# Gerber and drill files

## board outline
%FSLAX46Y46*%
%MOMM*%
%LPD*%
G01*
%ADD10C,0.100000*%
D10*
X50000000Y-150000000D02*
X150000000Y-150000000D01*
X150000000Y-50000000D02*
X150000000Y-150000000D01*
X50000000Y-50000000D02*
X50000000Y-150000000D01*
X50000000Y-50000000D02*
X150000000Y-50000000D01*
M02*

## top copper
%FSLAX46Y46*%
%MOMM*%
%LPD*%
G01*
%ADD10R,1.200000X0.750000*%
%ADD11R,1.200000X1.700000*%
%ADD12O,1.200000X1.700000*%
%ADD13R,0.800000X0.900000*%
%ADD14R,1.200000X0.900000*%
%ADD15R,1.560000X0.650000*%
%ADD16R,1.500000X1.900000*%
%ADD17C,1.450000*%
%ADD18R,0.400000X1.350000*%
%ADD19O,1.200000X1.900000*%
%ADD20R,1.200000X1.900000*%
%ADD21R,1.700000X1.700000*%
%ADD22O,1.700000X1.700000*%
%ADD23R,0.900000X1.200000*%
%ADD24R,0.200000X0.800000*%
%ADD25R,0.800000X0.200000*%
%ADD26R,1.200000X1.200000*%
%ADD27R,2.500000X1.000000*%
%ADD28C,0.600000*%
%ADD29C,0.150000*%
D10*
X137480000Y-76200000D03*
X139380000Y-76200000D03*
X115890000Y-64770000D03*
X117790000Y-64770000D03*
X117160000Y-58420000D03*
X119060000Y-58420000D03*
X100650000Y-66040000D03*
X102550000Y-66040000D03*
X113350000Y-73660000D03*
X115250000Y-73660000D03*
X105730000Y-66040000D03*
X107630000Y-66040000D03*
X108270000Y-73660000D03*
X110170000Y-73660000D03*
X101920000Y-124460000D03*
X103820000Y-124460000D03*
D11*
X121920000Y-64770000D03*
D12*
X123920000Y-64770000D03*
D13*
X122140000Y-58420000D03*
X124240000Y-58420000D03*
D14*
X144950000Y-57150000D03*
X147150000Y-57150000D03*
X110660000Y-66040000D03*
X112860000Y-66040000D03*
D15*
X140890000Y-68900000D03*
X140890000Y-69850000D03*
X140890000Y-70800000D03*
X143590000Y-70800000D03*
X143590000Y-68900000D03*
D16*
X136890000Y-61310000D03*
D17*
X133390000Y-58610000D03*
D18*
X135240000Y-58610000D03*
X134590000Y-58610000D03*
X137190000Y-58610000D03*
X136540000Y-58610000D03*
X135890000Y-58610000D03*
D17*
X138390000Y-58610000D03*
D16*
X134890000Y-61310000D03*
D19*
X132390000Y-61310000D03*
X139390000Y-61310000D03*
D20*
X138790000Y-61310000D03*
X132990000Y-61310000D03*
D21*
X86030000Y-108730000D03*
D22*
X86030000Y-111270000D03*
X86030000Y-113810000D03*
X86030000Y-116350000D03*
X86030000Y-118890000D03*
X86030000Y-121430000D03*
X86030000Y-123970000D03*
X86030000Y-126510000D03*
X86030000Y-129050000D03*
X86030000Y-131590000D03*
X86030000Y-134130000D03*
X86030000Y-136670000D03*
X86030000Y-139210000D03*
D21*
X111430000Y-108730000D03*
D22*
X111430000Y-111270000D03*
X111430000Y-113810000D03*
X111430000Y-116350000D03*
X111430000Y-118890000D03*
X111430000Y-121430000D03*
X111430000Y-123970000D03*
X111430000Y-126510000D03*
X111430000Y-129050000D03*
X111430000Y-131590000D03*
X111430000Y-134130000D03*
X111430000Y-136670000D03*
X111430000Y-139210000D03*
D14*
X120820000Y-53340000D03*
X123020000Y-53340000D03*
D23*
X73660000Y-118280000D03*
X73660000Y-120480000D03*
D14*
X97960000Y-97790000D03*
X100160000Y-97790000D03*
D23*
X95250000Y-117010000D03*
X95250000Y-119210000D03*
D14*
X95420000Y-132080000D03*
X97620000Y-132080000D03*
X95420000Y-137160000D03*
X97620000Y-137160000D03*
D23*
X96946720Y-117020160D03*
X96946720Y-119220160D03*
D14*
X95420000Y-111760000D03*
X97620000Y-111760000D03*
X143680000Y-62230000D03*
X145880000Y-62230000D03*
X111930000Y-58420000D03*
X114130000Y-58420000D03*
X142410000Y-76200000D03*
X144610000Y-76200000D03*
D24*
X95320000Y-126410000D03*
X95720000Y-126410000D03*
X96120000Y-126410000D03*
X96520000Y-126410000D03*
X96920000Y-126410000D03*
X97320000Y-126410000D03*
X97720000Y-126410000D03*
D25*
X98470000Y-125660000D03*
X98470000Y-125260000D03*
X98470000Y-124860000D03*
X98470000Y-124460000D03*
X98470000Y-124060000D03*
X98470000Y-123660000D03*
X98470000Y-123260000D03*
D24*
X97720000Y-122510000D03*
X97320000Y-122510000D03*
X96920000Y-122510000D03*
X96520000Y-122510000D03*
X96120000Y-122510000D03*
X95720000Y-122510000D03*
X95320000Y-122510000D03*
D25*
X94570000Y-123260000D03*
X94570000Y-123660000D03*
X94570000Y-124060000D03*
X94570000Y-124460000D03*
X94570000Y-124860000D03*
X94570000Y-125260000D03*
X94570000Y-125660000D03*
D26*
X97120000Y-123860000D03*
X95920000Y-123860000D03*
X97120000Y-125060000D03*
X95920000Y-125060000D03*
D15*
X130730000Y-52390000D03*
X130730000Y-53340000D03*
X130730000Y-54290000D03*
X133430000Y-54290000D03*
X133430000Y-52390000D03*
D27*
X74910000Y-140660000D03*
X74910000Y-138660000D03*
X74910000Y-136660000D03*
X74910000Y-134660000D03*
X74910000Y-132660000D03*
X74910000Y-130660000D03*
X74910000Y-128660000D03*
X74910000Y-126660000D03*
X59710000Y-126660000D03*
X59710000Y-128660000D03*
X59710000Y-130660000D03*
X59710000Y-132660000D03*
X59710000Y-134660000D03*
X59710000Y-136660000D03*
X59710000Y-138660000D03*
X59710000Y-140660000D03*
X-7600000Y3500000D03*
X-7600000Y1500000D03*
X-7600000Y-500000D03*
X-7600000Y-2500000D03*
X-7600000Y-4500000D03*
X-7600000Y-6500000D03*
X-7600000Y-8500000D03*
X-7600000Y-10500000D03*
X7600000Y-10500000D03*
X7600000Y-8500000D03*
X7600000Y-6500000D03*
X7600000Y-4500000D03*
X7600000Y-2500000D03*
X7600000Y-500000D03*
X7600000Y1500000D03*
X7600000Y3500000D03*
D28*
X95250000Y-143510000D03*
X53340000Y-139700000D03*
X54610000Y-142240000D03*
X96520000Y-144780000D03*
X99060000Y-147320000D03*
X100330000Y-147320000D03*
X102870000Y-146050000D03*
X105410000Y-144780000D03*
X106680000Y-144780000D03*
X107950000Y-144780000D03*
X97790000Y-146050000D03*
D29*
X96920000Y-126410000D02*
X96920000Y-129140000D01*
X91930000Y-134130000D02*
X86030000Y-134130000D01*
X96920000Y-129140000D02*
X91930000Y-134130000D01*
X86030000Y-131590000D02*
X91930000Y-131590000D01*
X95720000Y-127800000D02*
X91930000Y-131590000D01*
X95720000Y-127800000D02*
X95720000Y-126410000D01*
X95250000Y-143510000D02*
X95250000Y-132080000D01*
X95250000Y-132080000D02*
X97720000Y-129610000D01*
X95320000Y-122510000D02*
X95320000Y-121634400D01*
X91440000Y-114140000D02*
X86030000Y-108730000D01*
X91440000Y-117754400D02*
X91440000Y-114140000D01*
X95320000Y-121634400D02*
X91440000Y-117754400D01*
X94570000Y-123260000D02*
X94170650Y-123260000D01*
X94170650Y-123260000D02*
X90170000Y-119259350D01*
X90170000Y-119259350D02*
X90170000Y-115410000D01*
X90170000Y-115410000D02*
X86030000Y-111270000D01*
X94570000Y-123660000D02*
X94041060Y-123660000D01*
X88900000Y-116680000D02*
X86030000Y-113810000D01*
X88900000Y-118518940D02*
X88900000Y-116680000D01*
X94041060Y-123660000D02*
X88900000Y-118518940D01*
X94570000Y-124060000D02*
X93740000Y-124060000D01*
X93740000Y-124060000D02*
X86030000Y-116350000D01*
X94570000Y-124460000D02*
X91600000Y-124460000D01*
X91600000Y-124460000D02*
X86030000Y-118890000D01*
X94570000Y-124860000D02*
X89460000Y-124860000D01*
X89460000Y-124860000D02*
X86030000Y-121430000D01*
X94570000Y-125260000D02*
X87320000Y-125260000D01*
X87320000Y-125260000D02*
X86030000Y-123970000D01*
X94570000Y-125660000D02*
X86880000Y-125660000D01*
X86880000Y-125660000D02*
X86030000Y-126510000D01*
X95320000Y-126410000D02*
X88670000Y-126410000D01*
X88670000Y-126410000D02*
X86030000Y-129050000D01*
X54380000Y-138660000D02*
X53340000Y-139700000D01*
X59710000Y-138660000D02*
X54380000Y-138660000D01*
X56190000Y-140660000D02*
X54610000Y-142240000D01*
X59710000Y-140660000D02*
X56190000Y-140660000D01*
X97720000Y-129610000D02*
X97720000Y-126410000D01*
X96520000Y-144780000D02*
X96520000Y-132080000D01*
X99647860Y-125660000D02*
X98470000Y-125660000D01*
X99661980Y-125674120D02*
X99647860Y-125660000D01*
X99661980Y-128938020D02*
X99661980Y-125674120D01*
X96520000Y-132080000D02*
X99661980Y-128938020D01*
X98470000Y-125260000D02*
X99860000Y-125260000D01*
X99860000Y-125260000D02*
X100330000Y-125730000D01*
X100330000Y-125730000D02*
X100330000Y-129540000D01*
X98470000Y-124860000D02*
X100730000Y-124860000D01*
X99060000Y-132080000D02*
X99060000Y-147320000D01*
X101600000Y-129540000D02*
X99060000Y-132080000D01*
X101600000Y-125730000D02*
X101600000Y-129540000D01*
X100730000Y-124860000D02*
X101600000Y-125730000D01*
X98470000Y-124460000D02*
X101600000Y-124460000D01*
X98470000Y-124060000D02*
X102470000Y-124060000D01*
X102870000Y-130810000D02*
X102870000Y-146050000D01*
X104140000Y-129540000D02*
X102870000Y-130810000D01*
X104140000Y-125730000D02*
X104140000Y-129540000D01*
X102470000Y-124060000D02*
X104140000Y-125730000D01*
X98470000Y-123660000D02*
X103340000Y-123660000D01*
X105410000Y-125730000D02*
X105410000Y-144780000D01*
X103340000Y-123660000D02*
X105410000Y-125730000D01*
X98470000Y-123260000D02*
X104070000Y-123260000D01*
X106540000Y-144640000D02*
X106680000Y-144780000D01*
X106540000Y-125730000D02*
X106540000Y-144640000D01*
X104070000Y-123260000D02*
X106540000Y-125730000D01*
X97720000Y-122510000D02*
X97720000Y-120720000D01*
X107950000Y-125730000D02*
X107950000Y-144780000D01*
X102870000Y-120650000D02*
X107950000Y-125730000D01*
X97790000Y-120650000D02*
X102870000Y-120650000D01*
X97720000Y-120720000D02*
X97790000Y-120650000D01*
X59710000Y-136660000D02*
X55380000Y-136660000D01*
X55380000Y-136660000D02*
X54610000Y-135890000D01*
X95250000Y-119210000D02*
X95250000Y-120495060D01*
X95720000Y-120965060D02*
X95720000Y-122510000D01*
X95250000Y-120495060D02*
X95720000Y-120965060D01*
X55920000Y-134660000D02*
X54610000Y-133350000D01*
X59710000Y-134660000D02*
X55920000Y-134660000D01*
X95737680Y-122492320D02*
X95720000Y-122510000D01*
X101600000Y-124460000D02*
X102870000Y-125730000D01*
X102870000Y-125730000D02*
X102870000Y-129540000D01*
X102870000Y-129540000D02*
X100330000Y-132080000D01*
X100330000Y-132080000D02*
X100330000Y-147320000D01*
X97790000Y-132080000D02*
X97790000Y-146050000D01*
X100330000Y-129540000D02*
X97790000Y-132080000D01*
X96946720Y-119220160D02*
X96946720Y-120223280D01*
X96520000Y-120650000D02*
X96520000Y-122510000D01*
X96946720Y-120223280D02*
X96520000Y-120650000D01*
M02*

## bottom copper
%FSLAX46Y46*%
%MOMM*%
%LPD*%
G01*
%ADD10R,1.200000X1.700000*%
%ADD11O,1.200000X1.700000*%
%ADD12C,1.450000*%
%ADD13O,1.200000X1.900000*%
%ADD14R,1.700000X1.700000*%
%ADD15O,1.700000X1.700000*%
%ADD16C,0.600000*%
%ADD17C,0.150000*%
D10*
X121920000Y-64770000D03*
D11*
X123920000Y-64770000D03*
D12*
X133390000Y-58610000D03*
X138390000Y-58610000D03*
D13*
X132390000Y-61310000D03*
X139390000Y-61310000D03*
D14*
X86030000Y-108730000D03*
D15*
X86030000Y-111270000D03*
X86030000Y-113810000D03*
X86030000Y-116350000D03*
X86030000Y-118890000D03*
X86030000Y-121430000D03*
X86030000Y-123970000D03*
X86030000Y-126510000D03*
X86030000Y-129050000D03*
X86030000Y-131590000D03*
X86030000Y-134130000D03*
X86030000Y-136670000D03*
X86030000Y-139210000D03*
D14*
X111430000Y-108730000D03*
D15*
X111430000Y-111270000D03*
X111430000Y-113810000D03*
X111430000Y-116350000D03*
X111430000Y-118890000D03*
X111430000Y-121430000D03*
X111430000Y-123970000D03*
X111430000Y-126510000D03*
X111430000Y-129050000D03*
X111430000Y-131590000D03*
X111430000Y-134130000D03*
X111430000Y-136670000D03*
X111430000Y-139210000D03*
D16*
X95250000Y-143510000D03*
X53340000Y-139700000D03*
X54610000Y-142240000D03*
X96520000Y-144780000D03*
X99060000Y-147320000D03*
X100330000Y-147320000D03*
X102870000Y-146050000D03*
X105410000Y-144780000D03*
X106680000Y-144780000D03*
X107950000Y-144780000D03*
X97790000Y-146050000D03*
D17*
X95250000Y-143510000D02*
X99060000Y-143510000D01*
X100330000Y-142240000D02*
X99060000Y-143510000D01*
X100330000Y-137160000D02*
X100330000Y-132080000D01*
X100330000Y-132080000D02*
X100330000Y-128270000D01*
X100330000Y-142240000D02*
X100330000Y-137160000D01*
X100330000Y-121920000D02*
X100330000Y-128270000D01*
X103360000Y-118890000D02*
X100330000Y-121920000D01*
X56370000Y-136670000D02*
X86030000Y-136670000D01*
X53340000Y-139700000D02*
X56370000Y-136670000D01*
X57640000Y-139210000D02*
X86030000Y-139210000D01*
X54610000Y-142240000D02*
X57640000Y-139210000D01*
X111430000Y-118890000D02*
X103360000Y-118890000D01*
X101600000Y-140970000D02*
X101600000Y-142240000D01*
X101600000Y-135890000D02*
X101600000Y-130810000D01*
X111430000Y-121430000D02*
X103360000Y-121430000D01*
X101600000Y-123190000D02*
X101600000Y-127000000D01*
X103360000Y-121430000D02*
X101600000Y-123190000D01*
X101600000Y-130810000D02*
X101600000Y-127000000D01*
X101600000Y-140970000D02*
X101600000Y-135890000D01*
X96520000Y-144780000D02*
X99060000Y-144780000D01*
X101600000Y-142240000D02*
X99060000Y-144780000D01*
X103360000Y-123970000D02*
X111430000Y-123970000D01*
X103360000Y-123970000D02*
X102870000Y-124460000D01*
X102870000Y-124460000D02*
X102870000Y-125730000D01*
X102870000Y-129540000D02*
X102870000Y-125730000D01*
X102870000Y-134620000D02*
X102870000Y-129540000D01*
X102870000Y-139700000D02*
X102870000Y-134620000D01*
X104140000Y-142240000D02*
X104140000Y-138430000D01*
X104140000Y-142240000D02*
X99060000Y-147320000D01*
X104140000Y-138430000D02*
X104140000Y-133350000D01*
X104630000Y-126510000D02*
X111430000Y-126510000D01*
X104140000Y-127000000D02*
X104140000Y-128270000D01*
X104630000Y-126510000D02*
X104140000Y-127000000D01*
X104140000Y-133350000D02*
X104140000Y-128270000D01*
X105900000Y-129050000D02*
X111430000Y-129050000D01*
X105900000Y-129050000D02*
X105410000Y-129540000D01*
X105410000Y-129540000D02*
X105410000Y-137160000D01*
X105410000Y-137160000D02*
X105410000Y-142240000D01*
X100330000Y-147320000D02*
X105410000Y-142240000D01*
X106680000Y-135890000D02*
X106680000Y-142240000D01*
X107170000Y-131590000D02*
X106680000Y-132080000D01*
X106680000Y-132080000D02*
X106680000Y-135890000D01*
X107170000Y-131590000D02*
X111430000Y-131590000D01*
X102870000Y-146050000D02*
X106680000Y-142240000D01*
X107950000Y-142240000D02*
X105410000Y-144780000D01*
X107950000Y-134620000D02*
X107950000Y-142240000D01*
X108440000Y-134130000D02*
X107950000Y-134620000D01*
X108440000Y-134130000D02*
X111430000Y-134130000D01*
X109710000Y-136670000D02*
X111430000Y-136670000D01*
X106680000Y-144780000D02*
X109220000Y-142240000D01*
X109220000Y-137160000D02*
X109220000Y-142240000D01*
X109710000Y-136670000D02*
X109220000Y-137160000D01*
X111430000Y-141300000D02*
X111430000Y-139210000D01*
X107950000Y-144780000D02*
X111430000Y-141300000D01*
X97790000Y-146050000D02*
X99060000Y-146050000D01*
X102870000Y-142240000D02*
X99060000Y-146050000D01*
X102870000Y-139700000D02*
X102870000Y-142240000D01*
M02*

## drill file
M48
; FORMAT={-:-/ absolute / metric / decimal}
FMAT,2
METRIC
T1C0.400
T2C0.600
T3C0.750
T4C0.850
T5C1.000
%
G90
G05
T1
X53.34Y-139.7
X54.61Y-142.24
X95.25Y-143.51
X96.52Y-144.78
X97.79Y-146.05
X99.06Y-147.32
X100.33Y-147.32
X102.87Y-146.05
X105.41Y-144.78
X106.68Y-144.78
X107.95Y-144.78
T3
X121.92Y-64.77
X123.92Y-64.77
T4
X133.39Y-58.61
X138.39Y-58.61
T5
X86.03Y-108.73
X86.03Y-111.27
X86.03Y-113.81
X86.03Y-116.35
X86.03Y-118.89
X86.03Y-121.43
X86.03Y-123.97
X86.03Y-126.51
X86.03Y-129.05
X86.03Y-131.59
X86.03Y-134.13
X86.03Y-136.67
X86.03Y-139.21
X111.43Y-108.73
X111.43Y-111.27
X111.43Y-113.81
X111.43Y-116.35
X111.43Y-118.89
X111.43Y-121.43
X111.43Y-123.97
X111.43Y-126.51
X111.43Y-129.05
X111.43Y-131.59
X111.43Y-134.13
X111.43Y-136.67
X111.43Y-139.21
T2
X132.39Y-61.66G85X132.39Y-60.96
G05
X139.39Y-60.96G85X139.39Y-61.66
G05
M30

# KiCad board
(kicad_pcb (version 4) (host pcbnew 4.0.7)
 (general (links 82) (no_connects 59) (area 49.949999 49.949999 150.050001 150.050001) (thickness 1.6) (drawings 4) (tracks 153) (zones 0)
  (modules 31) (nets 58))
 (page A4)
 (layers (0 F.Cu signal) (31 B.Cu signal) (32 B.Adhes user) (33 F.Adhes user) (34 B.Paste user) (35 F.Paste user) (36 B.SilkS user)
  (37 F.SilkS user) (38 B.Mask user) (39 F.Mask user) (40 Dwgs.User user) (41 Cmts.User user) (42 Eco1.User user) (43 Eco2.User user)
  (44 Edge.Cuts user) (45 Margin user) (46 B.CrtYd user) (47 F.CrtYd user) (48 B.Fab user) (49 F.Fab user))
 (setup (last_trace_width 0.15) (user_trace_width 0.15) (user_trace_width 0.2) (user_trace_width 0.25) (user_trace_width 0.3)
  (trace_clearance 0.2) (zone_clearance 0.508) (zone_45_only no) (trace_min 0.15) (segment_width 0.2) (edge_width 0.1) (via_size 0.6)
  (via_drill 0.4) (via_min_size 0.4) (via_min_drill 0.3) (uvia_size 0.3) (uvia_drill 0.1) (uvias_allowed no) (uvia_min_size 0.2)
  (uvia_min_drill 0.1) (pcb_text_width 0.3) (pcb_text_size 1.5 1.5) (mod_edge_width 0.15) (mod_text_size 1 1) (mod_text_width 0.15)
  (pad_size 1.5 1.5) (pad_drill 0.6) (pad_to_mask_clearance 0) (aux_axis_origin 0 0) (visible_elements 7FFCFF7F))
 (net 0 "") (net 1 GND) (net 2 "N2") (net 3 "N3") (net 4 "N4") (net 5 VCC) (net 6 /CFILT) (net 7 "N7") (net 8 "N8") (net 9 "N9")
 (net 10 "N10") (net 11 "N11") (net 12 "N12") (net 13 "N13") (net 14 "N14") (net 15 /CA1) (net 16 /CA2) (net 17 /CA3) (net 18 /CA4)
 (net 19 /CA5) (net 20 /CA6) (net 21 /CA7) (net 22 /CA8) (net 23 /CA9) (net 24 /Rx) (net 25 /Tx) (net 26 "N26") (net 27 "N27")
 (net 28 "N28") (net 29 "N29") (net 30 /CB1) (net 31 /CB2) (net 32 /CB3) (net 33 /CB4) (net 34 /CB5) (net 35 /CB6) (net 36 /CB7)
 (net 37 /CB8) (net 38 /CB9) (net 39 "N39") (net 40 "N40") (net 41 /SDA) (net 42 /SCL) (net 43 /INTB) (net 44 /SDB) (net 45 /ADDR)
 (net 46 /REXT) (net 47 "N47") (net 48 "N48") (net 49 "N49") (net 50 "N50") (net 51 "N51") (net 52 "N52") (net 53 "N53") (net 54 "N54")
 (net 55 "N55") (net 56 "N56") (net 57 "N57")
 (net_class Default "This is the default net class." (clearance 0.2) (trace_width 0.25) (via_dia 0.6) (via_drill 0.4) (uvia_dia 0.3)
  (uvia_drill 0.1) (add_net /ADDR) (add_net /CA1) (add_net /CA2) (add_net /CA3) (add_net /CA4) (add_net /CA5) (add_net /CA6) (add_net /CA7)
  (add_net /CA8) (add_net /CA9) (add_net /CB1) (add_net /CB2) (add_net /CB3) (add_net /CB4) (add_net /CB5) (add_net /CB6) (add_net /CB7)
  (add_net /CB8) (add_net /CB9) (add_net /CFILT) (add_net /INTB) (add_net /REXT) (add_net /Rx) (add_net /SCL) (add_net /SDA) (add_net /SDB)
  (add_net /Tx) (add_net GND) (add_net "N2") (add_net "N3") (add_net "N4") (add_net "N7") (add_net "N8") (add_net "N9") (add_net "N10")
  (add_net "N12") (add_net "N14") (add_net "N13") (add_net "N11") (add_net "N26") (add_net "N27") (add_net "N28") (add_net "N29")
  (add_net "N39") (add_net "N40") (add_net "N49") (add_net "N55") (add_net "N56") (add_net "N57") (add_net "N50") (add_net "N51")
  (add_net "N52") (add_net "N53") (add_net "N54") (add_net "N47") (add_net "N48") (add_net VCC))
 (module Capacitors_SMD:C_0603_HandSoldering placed (layer F.Cu) (at 138.43 76.2)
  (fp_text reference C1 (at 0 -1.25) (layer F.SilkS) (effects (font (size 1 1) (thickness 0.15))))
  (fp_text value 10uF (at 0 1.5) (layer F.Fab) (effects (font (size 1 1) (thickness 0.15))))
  (pad 1 smd rect (at -0.95 0) (size 1.2 0.75) (layers F.Cu F.Paste F.Mask) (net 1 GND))
  (pad 2 smd rect (at 0.95 0) (size 1.2 0.75) (layers F.Cu F.Paste F.Mask) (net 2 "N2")))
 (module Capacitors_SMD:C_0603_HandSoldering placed (layer F.Cu) (at 116.84 64.77)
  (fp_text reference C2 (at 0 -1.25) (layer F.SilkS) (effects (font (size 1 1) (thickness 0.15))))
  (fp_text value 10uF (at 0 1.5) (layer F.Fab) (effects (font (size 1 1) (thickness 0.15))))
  (pad 1 smd rect (at -0.95 0) (size 1.2 0.75) (layers F.Cu F.Paste F.Mask) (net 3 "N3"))
  (pad 2 smd rect (at 0.95 0) (size 1.2 0.75) (layers F.Cu F.Paste F.Mask) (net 1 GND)))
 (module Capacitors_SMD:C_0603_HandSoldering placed (layer F.Cu) (at 118.11 58.42)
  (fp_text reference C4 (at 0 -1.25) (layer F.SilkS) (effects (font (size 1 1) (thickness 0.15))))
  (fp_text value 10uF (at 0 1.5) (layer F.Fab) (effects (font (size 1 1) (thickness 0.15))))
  (pad 1 smd rect (at -0.95 0) (size 1.2 0.75) (layers F.Cu F.Paste F.Mask) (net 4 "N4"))
  (pad 2 smd rect (at 0.95 0) (size 1.2 0.75) (layers F.Cu F.Paste F.Mask) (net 1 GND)))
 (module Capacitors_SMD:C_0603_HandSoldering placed (layer F.Cu) (at 101.6 66.04)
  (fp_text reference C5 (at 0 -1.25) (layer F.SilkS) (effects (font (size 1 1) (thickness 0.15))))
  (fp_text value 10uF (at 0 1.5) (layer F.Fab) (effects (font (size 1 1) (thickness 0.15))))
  (pad 1 smd rect (at -0.95 0) (size 1.2 0.75) (layers F.Cu F.Paste F.Mask) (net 1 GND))
  (pad 2 smd rect (at 0.95 0) (size 1.2 0.75) (layers F.Cu F.Paste F.Mask) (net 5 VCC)))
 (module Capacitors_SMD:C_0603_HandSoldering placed (layer F.Cu) (at 114.3 73.66)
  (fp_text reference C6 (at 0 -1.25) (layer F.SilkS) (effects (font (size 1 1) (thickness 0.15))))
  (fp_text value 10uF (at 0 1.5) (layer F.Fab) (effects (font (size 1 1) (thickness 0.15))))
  (pad 1 smd rect (at -0.95 0) (size 1.2 0.75) (layers F.Cu F.Paste F.Mask) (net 5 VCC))
  (pad 2 smd rect (at 0.95 0) (size 1.2 0.75) (layers F.Cu F.Paste F.Mask) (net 1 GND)))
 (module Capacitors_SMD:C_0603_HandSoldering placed (layer F.Cu) (at 106.68 66.04)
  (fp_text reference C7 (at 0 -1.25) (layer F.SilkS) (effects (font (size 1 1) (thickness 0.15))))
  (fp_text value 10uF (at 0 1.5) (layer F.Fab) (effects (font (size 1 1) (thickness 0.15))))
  (pad 1 smd rect (at -0.95 0) (size 1.2 0.75) (layers F.Cu F.Paste F.Mask) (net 5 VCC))
  (pad 2 smd rect (at 0.95 0) (size 1.2 0.75) (layers F.Cu F.Paste F.Mask) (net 1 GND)))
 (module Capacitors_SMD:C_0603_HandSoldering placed (layer F.Cu) (at 109.22 73.66)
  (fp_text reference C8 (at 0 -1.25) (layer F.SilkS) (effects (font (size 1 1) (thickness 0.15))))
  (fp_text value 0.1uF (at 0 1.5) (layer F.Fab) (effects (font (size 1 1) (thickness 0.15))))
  (pad 1 smd rect (at -0.95 0) (size 1.2 0.75) (layers F.Cu F.Paste F.Mask) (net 5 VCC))
  (pad 2 smd rect (at 0.95 0) (size 1.2 0.75) (layers F.Cu F.Paste F.Mask) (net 1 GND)))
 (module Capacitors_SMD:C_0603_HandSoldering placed (layer F.Cu) (at 102.87 124.46)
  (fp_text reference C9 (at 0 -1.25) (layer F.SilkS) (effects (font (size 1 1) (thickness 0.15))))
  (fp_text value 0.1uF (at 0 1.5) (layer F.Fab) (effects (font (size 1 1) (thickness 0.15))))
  (pad 1 smd rect (at -0.95 0) (size 1.2 0.75) (layers F.Cu F.Paste F.Mask) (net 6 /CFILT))
  (pad 2 smd rect (at 0.95 0) (size 1.2 0.75) (layers F.Cu F.Paste F.Mask) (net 1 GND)))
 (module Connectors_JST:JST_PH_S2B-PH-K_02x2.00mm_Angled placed (layer F.Cu) (at 121.92 64.77)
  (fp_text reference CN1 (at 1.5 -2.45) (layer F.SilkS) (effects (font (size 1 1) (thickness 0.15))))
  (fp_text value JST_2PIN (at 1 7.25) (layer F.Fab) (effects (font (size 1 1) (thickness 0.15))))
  (pad 1 thru_hole rect (at 0 0) (size 1.2 1.7) (drill 0.75) (layers *.Cu *.Mask) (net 1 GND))
  (pad 2 thru_hole oval (at 2 0) (size 1.2 1.7) (drill 0.75) (layers *.Cu *.Mask) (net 3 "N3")))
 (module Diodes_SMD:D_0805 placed (layer F.Cu) (at 123.19 58.42)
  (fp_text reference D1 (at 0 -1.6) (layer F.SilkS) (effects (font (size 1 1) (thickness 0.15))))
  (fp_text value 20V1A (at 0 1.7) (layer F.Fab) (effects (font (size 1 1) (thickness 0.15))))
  (pad 1 smd rect (at -1.05 0) (size 0.8 0.9) (layers F.Cu F.Paste F.Mask) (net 4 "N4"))
  (pad 2 smd rect (at 1.05 0) (size 0.8 0.9) (layers F.Cu F.Paste F.Mask) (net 3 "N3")))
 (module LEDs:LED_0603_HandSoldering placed (layer F.Cu) (at 146.05 57.15)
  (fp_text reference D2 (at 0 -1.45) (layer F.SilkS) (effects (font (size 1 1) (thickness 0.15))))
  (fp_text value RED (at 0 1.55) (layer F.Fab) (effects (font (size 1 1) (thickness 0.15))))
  (pad 1 smd rect (at -1.1 0) (size 1.2 0.9) (layers F.Cu F.Paste F.Mask) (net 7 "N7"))
  (pad 2 smd rect (at 1.1 0) (size 1.2 0.9) (layers F.Cu F.Paste F.Mask) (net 2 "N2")))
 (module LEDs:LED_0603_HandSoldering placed (layer F.Cu) (at 111.76 66.04)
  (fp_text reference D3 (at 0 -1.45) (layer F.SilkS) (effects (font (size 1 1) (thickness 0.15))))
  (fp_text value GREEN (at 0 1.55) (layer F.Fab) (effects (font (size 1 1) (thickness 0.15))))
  (pad 1 smd rect (at -1.1 0) (size 1.2 0.9) (layers F.Cu F.Paste F.Mask) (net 1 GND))
  (pad 2 smd rect (at 1.1 0) (size 1.2 0.9) (layers F.Cu F.Paste F.Mask) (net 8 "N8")))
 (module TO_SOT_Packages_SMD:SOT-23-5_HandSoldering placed (layer F.Cu) (at 142.24 69.85)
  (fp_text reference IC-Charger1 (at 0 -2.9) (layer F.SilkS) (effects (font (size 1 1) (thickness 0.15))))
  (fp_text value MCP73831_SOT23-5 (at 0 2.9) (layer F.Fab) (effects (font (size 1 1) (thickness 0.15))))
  (pad 1 smd rect (at -1.35 -0.95) (size 1.56 0.65) (layers F.Cu F.Paste F.Mask) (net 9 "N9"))
  (pad 2 smd rect (at -1.35 0) (size 1.56 0.65) (layers F.Cu F.Paste F.Mask) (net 1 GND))
  (pad 3 smd rect (at -1.35 0.95) (size 1.56 0.65) (layers F.Cu F.Paste F.Mask) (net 3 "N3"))
  (pad 4 smd rect (at 1.35 0.95) (size 1.56 0.65) (layers F.Cu F.Paste F.Mask) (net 2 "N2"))
  (pad 5 smd rect (at 1.35 -0.95) (size 1.56 0.65) (layers F.Cu F.Paste F.Mask) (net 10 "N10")))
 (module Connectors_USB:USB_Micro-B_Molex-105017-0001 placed (layer F.Cu) (at 135.89 60.96)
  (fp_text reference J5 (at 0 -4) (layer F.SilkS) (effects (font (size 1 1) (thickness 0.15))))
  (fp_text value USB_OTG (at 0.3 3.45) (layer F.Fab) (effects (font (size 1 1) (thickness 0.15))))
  (pad 6 smd rect (at 1 0.35) (size 1.5 1.9) (layers F.Cu F.Paste F.Mask) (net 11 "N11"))
  (pad 6 thru_hole circle (at -2.5 -2.35) (size 1.45 1.45) (drill 0.85) (layers *.Cu *.Mask) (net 11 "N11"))
  (pad 2 smd rect (at -0.65 -2.35) (size 0.4 1.35) (layers F.Cu F.Paste F.Mask) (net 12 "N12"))
  (pad 1 smd rect (at -1.3 -2.35) (size 0.4 1.35) (layers F.Cu F.Paste F.Mask) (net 2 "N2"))
  (pad 5 smd rect (at 1.3 -2.35) (size 0.4 1.35) (layers F.Cu F.Paste F.Mask) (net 1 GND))
  (pad 4 smd rect (at 0.65 -2.35) (size 0.4 1.35) (layers F.Cu F.Paste F.Mask) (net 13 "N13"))
  (pad 3 smd rect (at 0 -2.35) (size 0.4 1.35) (layers F.Cu F.Paste F.Mask) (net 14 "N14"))
  (pad 6 thru_hole circle (at 2.5 -2.35) (size 1.45 1.45) (drill 0.85) (layers *.Cu *.Mask) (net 11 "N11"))
  (pad 6 smd rect (at -1 0.35) (size 1.5 1.9) (layers F.Cu F.Paste F.Mask) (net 11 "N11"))
  (pad 6 thru_hole oval (at -3.5 0.35 180) (size 1.2 1.9) (drill oval 0.6 1.3) (layers *.Cu *.Mask) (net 11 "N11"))
  (pad 6 thru_hole oval (at 3.5 0.35) (size 1.2 1.9) (drill oval 0.6 1.3) (layers *.Cu *.Mask) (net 11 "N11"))
  (pad 6 smd rect (at 2.9 0.35) (size 1.2 1.9) (layers F.Cu F.Mask) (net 11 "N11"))
  (pad 6 smd rect (at -2.9 0.35) (size 1.2 1.9) (layers F.Cu F.Mask) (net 11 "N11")))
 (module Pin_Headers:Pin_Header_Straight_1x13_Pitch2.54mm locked (layer F.Cu) (at 86.03 108.73)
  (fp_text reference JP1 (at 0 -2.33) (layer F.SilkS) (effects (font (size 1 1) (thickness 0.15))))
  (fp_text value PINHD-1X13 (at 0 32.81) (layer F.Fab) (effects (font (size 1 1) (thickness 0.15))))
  (pad 1 thru_hole rect (at 0 0) (size 1.7 1.7) (drill 1) (layers *.Cu *.Mask) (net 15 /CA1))
  (pad 2 thru_hole oval (at 0 2.54) (size 1.7 1.7) (drill 1) (layers *.Cu *.Mask) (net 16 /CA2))
  (pad 3 thru_hole oval (at 0 5.08) (size 1.7 1.7) (drill 1) (layers *.Cu *.Mask) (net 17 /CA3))
  (pad 4 thru_hole oval (at 0 7.62) (size 1.7 1.7) (drill 1) (layers *.Cu *.Mask) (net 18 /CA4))
  (pad 5 thru_hole oval (at 0 10.16) (size 1.7 1.7) (drill 1) (layers *.Cu *.Mask) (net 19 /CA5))
  (pad 6 thru_hole oval (at 0 12.7) (size 1.7 1.7) (drill 1) (layers *.Cu *.Mask) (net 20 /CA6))
  (pad 7 thru_hole oval (at 0 15.24) (size 1.7 1.7) (drill 1) (layers *.Cu *.Mask) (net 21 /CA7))
  (pad 8 thru_hole oval (at 0 17.78) (size 1.7 1.7) (drill 1) (layers *.Cu *.Mask) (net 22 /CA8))
  (pad 9 thru_hole oval (at 0 20.32) (size 1.7 1.7) (drill 1) (layers *.Cu *.Mask) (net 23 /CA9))
  (pad 10 thru_hole oval (at 0 22.86) (size 1.7 1.7) (drill 1) (layers *.Cu *.Mask) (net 5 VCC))
  (pad 11 thru_hole oval (at 0 25.4) (size 1.7 1.7) (drill 1) (layers *.Cu *.Mask) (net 1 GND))
  (pad 12 thru_hole oval (at 0 27.94) (size 1.7 1.7) (drill 1) (layers *.Cu *.Mask) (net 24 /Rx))
  (pad 13 thru_hole oval (at 0 30.48) (size 1.7 1.7) (drill 1) (layers *.Cu *.Mask) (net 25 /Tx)))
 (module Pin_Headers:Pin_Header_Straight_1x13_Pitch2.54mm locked (layer F.Cu) (at 111.43 108.73)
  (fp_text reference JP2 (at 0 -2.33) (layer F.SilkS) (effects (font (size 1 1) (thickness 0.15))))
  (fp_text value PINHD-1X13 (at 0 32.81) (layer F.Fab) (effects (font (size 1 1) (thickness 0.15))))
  (pad 1 thru_hole rect (at 0 0) (size 1.7 1.7) (drill 1) (layers *.Cu *.Mask) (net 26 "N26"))
  (pad 2 thru_hole oval (at 0 2.54) (size 1.7 1.7) (drill 1) (layers *.Cu *.Mask) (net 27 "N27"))
  (pad 3 thru_hole oval (at 0 5.08) (size 1.7 1.7) (drill 1) (layers *.Cu *.Mask) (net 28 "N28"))
  (pad 4 thru_hole oval (at 0 7.62) (size 1.7 1.7) (drill 1) (layers *.Cu *.Mask) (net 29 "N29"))
  (pad 5 thru_hole oval (at 0 10.16) (size 1.7 1.7) (drill 1) (layers *.Cu *.Mask) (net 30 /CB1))
  (pad 6 thru_hole oval (at 0 12.7) (size 1.7 1.7) (drill 1) (layers *.Cu *.Mask) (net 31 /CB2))
  (pad 7 thru_hole oval (at 0 15.24) (size 1.7 1.7) (drill 1) (layers *.Cu *.Mask) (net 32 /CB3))
  (pad 8 thru_hole oval (at 0 17.78) (size 1.7 1.7) (drill 1) (layers *.Cu *.Mask) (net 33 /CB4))
  (pad 9 thru_hole oval (at 0 20.32) (size 1.7 1.7) (drill 1) (layers *.Cu *.Mask) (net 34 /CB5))
  (pad 10 thru_hole oval (at 0 22.86) (size 1.7 1.7) (drill 1) (layers *.Cu *.Mask) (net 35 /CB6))
  (pad 11 thru_hole oval (at 0 25.4) (size 1.7 1.7) (drill 1) (layers *.Cu *.Mask) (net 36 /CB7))
  (pad 12 thru_hole oval (at 0 27.94) (size 1.7 1.7) (drill 1) (layers *.Cu *.Mask) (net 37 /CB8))
  (pad 13 thru_hole oval (at 0 30.48) (size 1.7 1.7) (drill 1) (layers *.Cu *.Mask) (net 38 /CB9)))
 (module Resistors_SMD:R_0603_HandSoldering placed (layer F.Cu) (at 121.92 53.34)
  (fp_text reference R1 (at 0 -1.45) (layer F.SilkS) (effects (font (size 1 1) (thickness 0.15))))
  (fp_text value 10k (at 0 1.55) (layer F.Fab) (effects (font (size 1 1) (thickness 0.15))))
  (pad 1 smd rect (at -1.1 0) (size 1.2 0.9) (layers F.Cu F.Paste F.Mask) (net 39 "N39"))
  (pad 2 smd rect (at 1.1 0) (size 1.2 0.9) (layers F.Cu F.Paste F.Mask) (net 4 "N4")))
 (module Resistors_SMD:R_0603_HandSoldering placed (layer F.Cu) (at 73.66 119.38 270)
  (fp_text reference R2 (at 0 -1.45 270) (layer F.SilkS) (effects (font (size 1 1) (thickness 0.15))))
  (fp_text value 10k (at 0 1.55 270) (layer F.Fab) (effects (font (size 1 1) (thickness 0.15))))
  (pad 1 smd rect (at -1.1 0 270) (size 1.2 0.9) (layers F.Cu F.Paste F.Mask) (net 5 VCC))
  (pad 2 smd rect (at 1.1 0 270) (size 1.2 0.9) (layers F.Cu F.Paste F.Mask) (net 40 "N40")))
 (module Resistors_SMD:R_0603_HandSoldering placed (layer F.Cu) (at 99.06 97.79)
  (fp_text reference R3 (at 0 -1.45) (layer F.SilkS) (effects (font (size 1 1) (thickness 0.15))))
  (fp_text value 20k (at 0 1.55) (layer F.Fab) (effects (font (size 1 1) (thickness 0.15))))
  (pad 1 smd rect (at -1.1 0) (size 1.2 0.9) (layers F.Cu F.Paste F.Mask) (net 5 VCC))
  (pad 2 smd rect (at 1.1 0) (size 1.2 0.9) (layers F.Cu F.Paste F.Mask) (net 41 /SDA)))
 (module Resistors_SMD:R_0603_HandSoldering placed (layer F.Cu) (at 95.25 118.11 270)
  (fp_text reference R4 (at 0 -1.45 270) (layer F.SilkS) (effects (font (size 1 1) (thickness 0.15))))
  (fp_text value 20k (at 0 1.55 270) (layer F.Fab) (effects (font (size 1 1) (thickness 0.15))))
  (pad 1 smd rect (at -1.1 0 270) (size 1.2 0.9) (layers F.Cu F.Paste F.Mask) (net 5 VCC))
  (pad 2 smd rect (at 1.1 0 270) (size 1.2 0.9) (layers F.Cu F.Paste F.Mask) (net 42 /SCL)))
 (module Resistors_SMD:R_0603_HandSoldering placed (layer F.Cu) (at 96.52 132.08)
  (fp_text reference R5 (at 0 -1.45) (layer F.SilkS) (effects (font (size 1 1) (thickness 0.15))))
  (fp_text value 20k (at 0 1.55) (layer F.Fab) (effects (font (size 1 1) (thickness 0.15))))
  (pad 1 smd rect (at -1.1 0) (size 1.2 0.9) (layers F.Cu F.Paste F.Mask) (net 5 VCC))
  (pad 2 smd rect (at 1.1 0) (size 1.2 0.9) (layers F.Cu F.Paste F.Mask) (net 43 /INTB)))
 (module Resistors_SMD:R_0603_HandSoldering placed (layer F.Cu) (at 96.52 137.16)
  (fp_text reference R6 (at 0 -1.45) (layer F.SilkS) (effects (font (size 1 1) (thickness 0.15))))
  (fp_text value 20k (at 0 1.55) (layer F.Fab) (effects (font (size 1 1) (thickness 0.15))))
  (pad 1 smd rect (at -1.1 0) (size 1.2 0.9) (layers F.Cu F.Paste F.Mask) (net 5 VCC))
  (pad 2 smd rect (at 1.1 0) (size 1.2 0.9) (layers F.Cu F.Paste F.Mask) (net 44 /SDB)))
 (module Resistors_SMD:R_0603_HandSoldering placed (layer F.Cu) (at 96.94672 118.12016 270)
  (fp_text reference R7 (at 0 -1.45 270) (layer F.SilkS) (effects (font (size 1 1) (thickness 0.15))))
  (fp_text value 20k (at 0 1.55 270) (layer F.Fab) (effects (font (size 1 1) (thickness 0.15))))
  (pad 1 smd rect (at -1.1 0 270) (size 1.2 0.9) (layers F.Cu F.Paste F.Mask) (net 1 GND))
  (pad 2 smd rect (at 1.1 0 270) (size 1.2 0.9) (layers F.Cu F.Paste F.Mask) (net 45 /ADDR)))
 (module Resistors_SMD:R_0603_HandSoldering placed (layer F.Cu) (at 96.52 111.76)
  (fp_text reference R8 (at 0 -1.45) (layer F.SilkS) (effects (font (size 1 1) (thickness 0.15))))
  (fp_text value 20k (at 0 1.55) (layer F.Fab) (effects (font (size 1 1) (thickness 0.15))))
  (pad 1 smd rect (at -1.1 0) (size 1.2 0.9) (layers F.Cu F.Paste F.Mask) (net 1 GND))
  (pad 2 smd rect (at 1.1 0) (size 1.2 0.9) (layers F.Cu F.Paste F.Mask) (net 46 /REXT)))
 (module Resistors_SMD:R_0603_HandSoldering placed (layer F.Cu) (at 144.78 62.23)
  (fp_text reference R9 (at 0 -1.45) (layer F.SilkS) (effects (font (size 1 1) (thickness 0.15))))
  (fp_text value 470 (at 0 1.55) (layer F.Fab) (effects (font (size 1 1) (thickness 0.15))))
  (pad 1 smd rect (at -1.1 0) (size 1.2 0.9) (layers F.Cu F.Paste F.Mask) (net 9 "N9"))
  (pad 2 smd rect (at 1.1 0) (size 1.2 0.9) (layers F.Cu F.Paste F.Mask) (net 7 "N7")))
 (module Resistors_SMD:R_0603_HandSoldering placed (layer F.Cu) (at 113.03 58.42)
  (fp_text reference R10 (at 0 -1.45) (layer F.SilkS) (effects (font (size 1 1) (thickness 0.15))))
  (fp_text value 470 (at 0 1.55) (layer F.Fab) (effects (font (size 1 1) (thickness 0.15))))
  (pad 1 smd rect (at -1.1 0) (size 1.2 0.9) (layers F.Cu F.Paste F.Mask) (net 9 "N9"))
  (pad 2 smd rect (at 1.1 0) (size 1.2 0.9) (layers F.Cu F.Paste F.Mask) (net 8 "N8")))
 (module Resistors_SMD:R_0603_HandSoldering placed (layer F.Cu) (at 143.51 76.2)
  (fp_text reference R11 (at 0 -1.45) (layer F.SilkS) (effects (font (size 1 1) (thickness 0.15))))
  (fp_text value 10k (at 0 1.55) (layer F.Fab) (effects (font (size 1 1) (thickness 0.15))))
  (pad 1 smd rect (at -1.1 0) (size 1.2 0.9) (layers F.Cu F.Paste F.Mask) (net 1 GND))
  (pad 2 smd rect (at 1.1 0) (size 1.2 0.9) (layers F.Cu F.Paste F.Mask) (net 10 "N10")))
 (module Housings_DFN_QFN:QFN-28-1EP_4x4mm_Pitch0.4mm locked (layer F.Cu) (at 96.52 124.46 90)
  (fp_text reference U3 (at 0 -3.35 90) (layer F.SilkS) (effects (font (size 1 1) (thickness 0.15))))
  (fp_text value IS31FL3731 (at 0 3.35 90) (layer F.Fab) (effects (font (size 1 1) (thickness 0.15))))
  (pad 1 smd rect (at -1.95 -1.2 90) (size 0.8 0.2) (layers F.Cu F.Paste F.Mask) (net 23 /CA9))
  (pad 2 smd rect (at -1.95 -0.8 90) (size 0.8 0.2) (layers F.Cu F.Paste F.Mask) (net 5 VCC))
  (pad 3 smd rect (at -1.95 -0.4 90) (size 0.8 0.2) (layers F.Cu F.Paste F.Mask) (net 44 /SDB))
  (pad 4 smd rect (at -1.95 0 90) (size 0.8 0.2) (layers F.Cu F.Paste F.Mask) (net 43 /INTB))
  (pad 5 smd rect (at -1.95 0.4 90) (size 0.8 0.2) (layers F.Cu F.Paste F.Mask) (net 1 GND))
  (pad 6 smd rect (at -1.95 0.8 90) (size 0.8 0.2) (layers F.Cu F.Paste F.Mask) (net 46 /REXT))
  (pad 7 smd rect (at -1.95 1.2 90) (size 0.8 0.2) (layers F.Cu F.Paste F.Mask) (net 30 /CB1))
  (pad 8 smd rect (at -1.2 1.95 180) (size 0.8 0.2) (layers F.Cu F.Paste F.Mask) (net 31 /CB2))
  (pad 9 smd rect (at -0.8 1.95 180) (size 0.8 0.2) (layers F.Cu F.Paste F.Mask) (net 32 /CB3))
  (pad 10 smd rect (at -0.4 1.95 180) (size 0.8 0.2) (layers F.Cu F.Paste F.Mask) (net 33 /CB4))
  (pad 11 smd rect (at 0 1.95 180) (size 0.8 0.2) (layers F.Cu F.Paste F.Mask) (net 34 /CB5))
  (pad 12 smd rect (at 0.4 1.95 180) (size 0.8 0.2) (layers F.Cu F.Paste F.Mask) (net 35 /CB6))
  (pad 13 smd rect (at 0.8 1.95 180) (size 0.8 0.2) (layers F.Cu F.Paste F.Mask) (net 36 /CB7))
  (pad 14 smd rect (at 1.2 1.95 180) (size 0.8 0.2) (layers F.Cu F.Paste F.Mask) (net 37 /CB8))
  (pad 15 smd rect (at 1.95 1.2 90) (size 0.8 0.2) (layers F.Cu F.Paste F.Mask) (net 38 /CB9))
  (pad 16 smd rect (at 1.95 0.8 90) (size 0.8 0.2) (layers F.Cu F.Paste F.Mask) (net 6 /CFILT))
  (pad 17 smd rect (at 1.95 0.4 90) (size 0.8 0.2) (layers F.Cu F.Paste F.Mask) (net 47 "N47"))
  (pad 18 smd rect (at 1.95 0 90) (size 0.8 0.2) (layers F.Cu F.Paste F.Mask) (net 45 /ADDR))
  (pad 19 smd rect (at 1.95 -0.4 90) (size 0.8 0.2) (layers F.Cu F.Paste F.Mask) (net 41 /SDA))
  (pad 20 smd rect (at 1.95 -0.8 90) (size 0.8 0.2) (layers F.Cu F.Paste F.Mask) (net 42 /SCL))
  (pad 21 smd rect (at 1.95 -1.2 90) (size 0.8 0.2) (layers F.Cu F.Paste F.Mask) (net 15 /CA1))
  (pad 22 smd rect (at 1.2 -1.95 180) (size 0.8 0.2) (layers F.Cu F.Paste F.Mask) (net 16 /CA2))
  (pad 23 smd rect (at 0.8 -1.95 180) (size 0.8 0.2) (layers F.Cu F.Paste F.Mask) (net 17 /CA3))
  (pad 24 smd rect (at 0.4 -1.95 180) (size 0.8 0.2) (layers F.Cu F.Paste F.Mask) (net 18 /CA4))
  (pad 25 smd rect (at 0 -1.95 180) (size 0.8 0.2) (layers F.Cu F.Paste F.Mask) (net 19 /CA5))
  (pad 26 smd rect (at -0.4 -1.95 180) (size 0.8 0.2) (layers F.Cu F.Paste F.Mask) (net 20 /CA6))
  (pad 27 smd rect (at -0.8 -1.95 180) (size 0.8 0.2) (layers F.Cu F.Paste F.Mask) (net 21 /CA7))
  (pad 28 smd rect (at -1.2 -1.95 180) (size 0.8 0.2) (layers F.Cu F.Paste F.Mask) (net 22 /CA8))
  (pad 29 smd rect (at 0.6 0.6 90) (size 1.2 1.2) (layers F.Cu F.Paste F.Mask) (solder_paste_margin_ratio -0.2))
  (pad 29 smd rect (at 0.6 -0.6 90) (size 1.2 1.2) (layers F.Cu F.Paste F.Mask) (solder_paste_margin_ratio -0.2))
  (pad 29 smd rect (at -0.6 0.6 90) (size 1.2 1.2) (layers F.Cu F.Paste F.Mask) (solder_paste_margin_ratio -0.2))
  (pad 29 smd rect (at -0.6 -0.6 90) (size 1.2 1.2) (layers F.Cu F.Paste F.Mask) (solder_paste_margin_ratio -0.2)))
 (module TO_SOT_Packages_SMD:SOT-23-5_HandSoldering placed (layer F.Cu) (at 132.08 53.34)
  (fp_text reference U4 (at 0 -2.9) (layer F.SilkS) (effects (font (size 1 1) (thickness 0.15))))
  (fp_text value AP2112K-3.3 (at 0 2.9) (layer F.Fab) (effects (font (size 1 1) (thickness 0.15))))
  (pad 1 smd rect (at -1.35 -0.95) (size 1.56 0.65) (layers F.Cu F.Paste F.Mask) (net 4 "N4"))
  (pad 2 smd rect (at -1.35 0) (size 1.56 0.65) (layers F.Cu F.Paste F.Mask) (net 1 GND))
  (pad 3 smd rect (at -1.35 0.95) (size 1.56 0.65) (layers F.Cu F.Paste F.Mask) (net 39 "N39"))
  (pad 4 smd rect (at 1.35 0.95) (size 1.56 0.65) (layers F.Cu F.Paste F.Mask) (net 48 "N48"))
  (pad 5 smd rect (at 1.35 -0.95) (size 1.56 0.65) (layers F.Cu F.Paste F.Mask) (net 5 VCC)))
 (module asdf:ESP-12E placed (layer F.Cu) (at 67.31 137.16 180)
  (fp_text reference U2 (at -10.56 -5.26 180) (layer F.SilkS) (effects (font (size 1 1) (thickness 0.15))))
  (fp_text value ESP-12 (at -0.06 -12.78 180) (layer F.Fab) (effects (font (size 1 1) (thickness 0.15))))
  (pad 1 smd rect (at -7.6 -3.5 180) (size 2.5 1) (layers F.Cu F.Paste F.Mask) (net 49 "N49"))
  (pad 2 smd rect (at -7.6 -1.5 180) (size 2.5 1) (layers F.Cu F.Paste F.Mask) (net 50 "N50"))
  (pad 3 smd rect (at -7.6 0.5 180) (size 2.5 1) (layers F.Cu F.Paste F.Mask) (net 40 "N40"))
  (pad 4 smd rect (at -7.6 2.5 180) (size 2.5 1) (layers F.Cu F.Paste F.Mask) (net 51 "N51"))
  (pad 5 smd rect (at -7.6 4.5 180) (size 2.5 1) (layers F.Cu F.Paste F.Mask) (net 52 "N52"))
  (pad 6 smd rect (at -7.6 6.5 180) (size 2.5 1) (layers F.Cu F.Paste F.Mask) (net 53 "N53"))
  (pad 7 smd rect (at -7.6 8.5 180) (size 2.5 1) (layers F.Cu F.Paste F.Mask) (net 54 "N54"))
  (pad 8 smd rect (at -7.6 10.5 180) (size 2.5 1) (layers F.Cu F.Paste F.Mask) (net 5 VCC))
  (pad 9 smd rect (at 7.6 10.5 180) (size 2.5 1) (layers F.Cu F.Paste F.Mask) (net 1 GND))
  (pad 10 smd rect (at 7.6 8.5 180) (size 2.5 1) (layers F.Cu F.Paste F.Mask) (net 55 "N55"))
  (pad 11 smd rect (at 7.6 6.5 180) (size 2.5 1) (layers F.Cu F.Paste F.Mask) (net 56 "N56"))
  (pad 12 smd rect (at 7.6 4.5 180) (size 2.5 1) (layers F.Cu F.Paste F.Mask) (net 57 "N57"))
  (pad 13 smd rect (at 7.6 2.5 180) (size 2.5 1) (layers F.Cu F.Paste F.Mask) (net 42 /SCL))
  (pad 14 smd rect (at 7.6 0.5 180) (size 2.5 1) (layers F.Cu F.Paste F.Mask) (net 41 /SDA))
  (pad 15 smd rect (at 7.6 -1.5 180) (size 2.5 1) (layers F.Cu F.Paste F.Mask) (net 24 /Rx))
  (pad 16 smd rect (at 7.6 -3.5 180) (size 2.5 1) (layers F.Cu F.Paste F.Mask) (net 25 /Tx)))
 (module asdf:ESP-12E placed (layer F.Cu) (at 0 0)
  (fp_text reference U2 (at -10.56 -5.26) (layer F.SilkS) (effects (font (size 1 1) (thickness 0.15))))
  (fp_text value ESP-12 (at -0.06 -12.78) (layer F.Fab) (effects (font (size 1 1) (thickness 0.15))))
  (pad 1 smd rect (at -7.6 -3.5) (size 2.5 1) (layers F.Cu F.Paste F.Mask))
  (pad 2 smd rect (at -7.6 -1.5) (size 2.5 1) (layers F.Cu F.Paste F.Mask))
  (pad 3 smd rect (at -7.6 0.5) (size 2.5 1) (layers F.Cu F.Paste F.Mask))
  (pad 4 smd rect (at -7.6 2.5) (size 2.5 1) (layers F.Cu F.Paste F.Mask))
  (pad 5 smd rect (at -7.6 4.5) (size 2.5 1) (layers F.Cu F.Paste F.Mask))
  (pad 6 smd rect (at -7.6 6.5) (size 2.5 1) (layers F.Cu F.Paste F.Mask))
  (pad 7 smd rect (at -7.6 8.5) (size 2.5 1) (layers F.Cu F.Paste F.Mask))
  (pad 8 smd rect (at -7.6 10.5) (size 2.5 1) (layers F.Cu F.Paste F.Mask))
  (pad 9 smd rect (at 7.6 10.5) (size 2.5 1) (layers F.Cu F.Paste F.Mask))
  (pad 10 smd rect (at 7.6 8.5) (size 2.5 1) (layers F.Cu F.Paste F.Mask))
  (pad 11 smd rect (at 7.6 6.5) (size 2.5 1) (layers F.Cu F.Paste F.Mask))
  (pad 12 smd rect (at 7.6 4.5) (size 2.5 1) (layers F.Cu F.Paste F.Mask))
  (pad 13 smd rect (at 7.6 2.5) (size 2.5 1) (layers F.Cu F.Paste F.Mask))
  (pad 14 smd rect (at 7.6 0.5) (size 2.5 1) (layers F.Cu F.Paste F.Mask))
  (pad 15 smd rect (at 7.6 -1.5) (size 2.5 1) (layers F.Cu F.Paste F.Mask))
  (pad 16 smd rect (at 7.6 -3.5) (size 2.5 1) (layers F.Cu F.Paste F.Mask)))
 (gr_line (start 50 150) (end 150 150) (angle 90) (layer Edge.Cuts) (width 0.1))
 (gr_line (start 150 50) (end 150 150) (angle 90) (layer Edge.Cuts) (width 0.1))
 (gr_line (start 50 50) (end 50 150) (angle 90) (layer Edge.Cuts) (width 0.1))
 (gr_line (start 50 50) (end 150 50) (angle 90) (layer Edge.Cuts) (width 0.1))
 (segment (start 96.92 126.41) (end 96.92 129.14) (width 0.15) (layer F.Cu) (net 1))
 (segment (start 91.93 134.13) (end 86.03 134.13) (width 0.15) (layer F.Cu) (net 1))
 (segment (start 96.92 129.14) (end 91.93 134.13) (width 0.15) (layer F.Cu) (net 1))
 (segment (start 86.03 131.59) (end 91.93 131.59) (width 0.15) (layer F.Cu) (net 5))
 (segment (start 95.72 127.8) (end 91.93 131.59) (width 0.15) (layer F.Cu) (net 5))
 (segment (start 95.72 127.8) (end 95.72 126.41) (width 0.15) (layer F.Cu) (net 5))
 (segment (start 95.25 143.51) (end 95.25 132.08) (width 0.15) (layer F.Cu) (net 5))
 (segment (start 95.25 143.51) (end 99.06 143.51) (width 0.15) (layer B.Cu) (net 5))
 (via (at 95.25 143.51) (size 0.6) (drill 0.4) (layers F.Cu B.Cu) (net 5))
 (segment (start 95.25 132.08) (end 97.72 129.61) (width 0.15) (layer F.Cu) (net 5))
 (segment (start 100.33 142.24) (end 99.06 143.51) (width 0.15) (layer B.Cu) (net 5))
 (segment (start 100.33 137.16) (end 100.33 132.08) (width 0.15) (layer B.Cu) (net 5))
 (segment (start 100.33 132.08) (end 100.33 128.27) (width 0.15) (layer B.Cu) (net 5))
 (segment (start 100.33 142.24) (end 100.33 137.16) (width 0.15) (layer B.Cu) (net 5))
 (segment (start 100.33 121.92) (end 100.33 128.27) (width 0.15) (layer B.Cu) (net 5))
 (segment (start 103.36 118.89) (end 100.33 121.92) (width 0.15) (layer B.Cu) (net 5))
 (segment (start 95.32 122.51) (end 95.32 121.6344) (width 0.15) (layer F.Cu) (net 15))
 (segment (start 91.44 114.14) (end 86.03 108.73) (width 0.15) (layer F.Cu) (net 15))
 (segment (start 91.44 117.7544) (end 91.44 114.14) (width 0.15) (layer F.Cu) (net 15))
 (segment (start 95.32 121.6344) (end 91.44 117.7544) (width 0.15) (layer F.Cu) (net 15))
 (segment (start 94.57 123.26) (end 94.17065 123.26) (width 0.15) (layer F.Cu) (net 16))
 (segment (start 94.17065 123.26) (end 90.17 119.25935) (width 0.15) (layer F.Cu) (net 16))
 (segment (start 90.17 119.25935) (end 90.17 115.41) (width 0.15) (layer F.Cu) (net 16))
 (segment (start 90.17 115.41) (end 86.03 111.27) (width 0.15) (layer F.Cu) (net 16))
 (segment (start 94.57 123.66) (end 94.04106 123.66) (width 0.15) (layer F.Cu) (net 17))
 (segment (start 88.9 116.68) (end 86.03 113.81) (width 0.15) (layer F.Cu) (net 17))
 (segment (start 88.9 118.51894) (end 88.9 116.68) (width 0.15) (layer F.Cu) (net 17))
 (segment (start 94.04106 123.66) (end 88.9 118.51894) (width 0.15) (layer F.Cu) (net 17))
 (segment (start 94.57 124.06) (end 93.74 124.06) (width 0.15) (layer F.Cu) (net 18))
 (segment (start 93.74 124.06) (end 86.03 116.35) (width 0.15) (layer F.Cu) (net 18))
 (segment (start 94.57 124.46) (end 91.6 124.46) (width 0.15) (layer F.Cu) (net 19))
 (segment (start 91.6 124.46) (end 86.03 118.89) (width 0.15) (layer F.Cu) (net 19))
 (segment (start 94.57 124.86) (end 89.46 124.86) (width 0.15) (layer F.Cu) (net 20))
 (segment (start 89.46 124.86) (end 86.03 121.43) (width 0.15) (layer F.Cu) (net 20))
 (segment (start 94.57 125.26) (end 87.32 125.26) (width 0.15) (layer F.Cu) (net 21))
 (segment (start 87.32 125.26) (end 86.03 123.97) (width 0.15) (layer F.Cu) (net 21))
 (segment (start 94.57 125.66) (end 86.88 125.66) (width 0.15) (layer F.Cu) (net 22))
 (segment (start 86.88 125.66) (end 86.03 126.51) (width 0.15) (layer F.Cu) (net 22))
 (segment (start 95.32 126.41) (end 88.67 126.41) (width 0.15) (layer F.Cu) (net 23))
 (segment (start 88.67 126.41) (end 86.03 129.05) (width 0.15) (layer F.Cu) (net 23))
 (via (at 53.34 139.7) (size 0.6) (drill 0.4) (layers F.Cu B.Cu) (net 24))
 (segment (start 54.38 138.66) (end 53.34 139.7) (width 0.15) (layer F.Cu) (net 24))
 (segment (start 59.71 138.66) (end 54.38 138.66) (width 0.15) (layer F.Cu) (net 24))
 (segment (start 56.37 136.67) (end 86.03 136.67) (width 0.15) (layer B.Cu) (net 24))
 (segment (start 53.34 139.7) (end 56.37 136.67) (width 0.15) (layer B.Cu) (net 24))
 (via (at 54.61 142.24) (size 0.6) (drill 0.4) (layers F.Cu B.Cu) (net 25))
 (segment (start 56.19 140.66) (end 54.61 142.24) (width 0.15) (layer F.Cu) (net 25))
 (segment (start 59.71 140.66) (end 56.19 140.66) (width 0.15) (layer F.Cu) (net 25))
 (segment (start 57.64 139.21) (end 86.03 139.21) (width 0.15) (layer B.Cu) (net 25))
 (segment (start 54.61 142.24) (end 57.64 139.21) (width 0.15) (layer B.Cu) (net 25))
 (segment (start 111.43 118.89) (end 103.36 118.89) (width 0.15) (layer B.Cu) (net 30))
 (segment (start 97.72 129.61) (end 97.72 126.41) (width 0.15) (layer F.Cu) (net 30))
 (segment (start 96.52 144.78) (end 96.52 132.08) (width 0.15) (layer F.Cu) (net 31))
 (segment (start 101.6 140.97) (end 101.6 142.24) (width 0.15) (layer B.Cu) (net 31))
 (segment (start 101.6 135.89) (end 101.6 130.81) (width 0.15) (layer B.Cu) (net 31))
 (segment (start 111.43 121.43) (end 103.36 121.43) (width 0.15) (layer B.Cu) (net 31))
 (segment (start 101.6 123.19) (end 101.6 127) (width 0.15) (layer B.Cu) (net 31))
 (segment (start 103.36 121.43) (end 101.6 123.19) (width 0.15) (layer B.Cu) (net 31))
 (segment (start 101.6 130.81) (end 101.6 127) (width 0.15) (layer B.Cu) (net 31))
 (segment (start 101.6 140.97) (end 101.6 135.89) (width 0.15) (layer B.Cu) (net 31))
 (segment (start 96.52 144.78) (end 99.06 144.78) (width 0.15) (layer B.Cu) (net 31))
 (segment (start 101.6 142.24) (end 99.06 144.78) (width 0.15) (layer B.Cu) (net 31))
 (via (at 96.52 144.78) (size 0.6) (drill 0.4) (layers F.Cu B.Cu) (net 31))
 (segment (start 99.64786 125.66) (end 98.47 125.66) (width 0.15) (layer F.Cu) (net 31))
 (segment (start 99.66198 125.67412) (end 99.64786 125.66) (width 0.15) (layer F.Cu) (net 31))
 (segment (start 99.66198 128.93802) (end 99.66198 125.67412) (width 0.15) (layer F.Cu) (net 31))
 (segment (start 96.52 132.08) (end 99.66198 128.93802) (width 0.15) (layer F.Cu) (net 31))
 (segment (start 98.47 125.26) (end 99.86 125.26) (width 0.15) (layer F.Cu) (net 32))
 (segment (start 103.36 123.97) (end 111.43 123.97) (width 0.15) (layer B.Cu) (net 32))
 (segment (start 99.86 125.26) (end 100.33 125.73) (width 0.15) (layer F.Cu) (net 32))
 (segment (start 103.36 123.97) (end 102.87 124.46) (width 0.15) (layer B.Cu) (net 32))
 (segment (start 100.33 125.73) (end 100.33 129.54) (width 0.15) (layer F.Cu) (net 32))
 (segment (start 102.87 124.46) (end 102.87 125.73) (width 0.15) (layer B.Cu) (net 32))
 (segment (start 102.87 129.54) (end 102.87 125.73) (width 0.15) (layer B.Cu) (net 32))
 (segment (start 102.87 134.62) (end 102.87 129.54) (width 0.15) (layer B.Cu) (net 32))
 (segment (start 102.87 139.7) (end 102.87 134.62) (width 0.15) (layer B.Cu) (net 32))
 (segment (start 98.47 124.86) (end 100.73 124.86) (width 0.15) (layer F.Cu) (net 33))
 (segment (start 104.14 142.24) (end 104.14 138.43) (width 0.15) (layer B.Cu) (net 33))
 (segment (start 104.14 142.24) (end 99.06 147.32) (width 0.15) (layer B.Cu) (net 33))
 (segment (start 104.14 138.43) (end 104.14 133.35) (width 0.15) (layer B.Cu) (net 33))
 (segment (start 104.63 126.51) (end 111.43 126.51) (width 0.15) (layer B.Cu) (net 33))
 (segment (start 104.14 127) (end 104.14 128.27) (width 0.15) (layer B.Cu) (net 33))
 (segment (start 104.63 126.51) (end 104.14 127) (width 0.15) (layer B.Cu) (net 33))
 (segment (start 104.14 133.35) (end 104.14 128.27) (width 0.15) (layer B.Cu) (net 33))
 (via (at 99.06 147.32) (size 0.6) (drill 0.4) (layers F.Cu B.Cu) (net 33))
 (segment (start 99.06 132.08) (end 99.06 147.32) (width 0.15) (layer F.Cu) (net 33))
 (segment (start 101.6 129.54) (end 99.06 132.08) (width 0.15) (layer F.Cu) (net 33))
 (segment (start 101.6 125.73) (end 101.6 129.54) (width 0.15) (layer F.Cu) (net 33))
 (segment (start 100.73 124.86) (end 101.6 125.73) (width 0.15) (layer F.Cu) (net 33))
 (segment (start 98.47 124.46) (end 101.6 124.46) (width 0.15) (layer F.Cu) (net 34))
 (segment (start 105.9 129.05) (end 111.43 129.05) (width 0.15) (layer B.Cu) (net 34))
 (segment (start 105.9 129.05) (end 105.41 129.54) (width 0.15) (layer B.Cu) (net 34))
 (segment (start 105.41 129.54) (end 105.41 137.16) (width 0.15) (layer B.Cu) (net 34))
 (segment (start 105.41 137.16) (end 105.41 142.24) (width 0.15) (layer B.Cu) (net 34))
 (segment (start 100.33 147.32) (end 105.41 142.24) (width 0.15) (layer B.Cu) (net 34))
 (via (at 100.33 147.32) (size 0.6) (drill 0.4) (layers F.Cu B.Cu) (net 34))
 (segment (start 98.47 124.06) (end 102.47 124.06) (width 0.15) (layer F.Cu) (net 35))
 (segment (start 106.68 135.89) (end 106.68 142.24) (width 0.15) (layer B.Cu) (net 35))
 (segment (start 107.17 131.59) (end 106.68 132.08) (width 0.15) (layer B.Cu) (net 35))
 (segment (start 106.68 132.08) (end 106.68 135.89) (width 0.15) (layer B.Cu) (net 35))
 (segment (start 107.17 131.59) (end 111.43 131.59) (width 0.15) (layer B.Cu) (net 35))
 (segment (start 102.87 146.05) (end 106.68 142.24) (width 0.15) (layer B.Cu) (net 35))
 (via (at 102.87 146.05) (size 0.6) (drill 0.4) (layers F.Cu B.Cu) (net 35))
 (segment (start 102.87 130.81) (end 102.87 146.05) (width 0.15) (layer F.Cu) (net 35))
 (segment (start 104.14 129.54) (end 102.87 130.81) (width 0.15) (layer F.Cu) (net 35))
 (segment (start 104.14 125.73) (end 104.14 129.54) (width 0.15) (layer F.Cu) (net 35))
 (segment (start 102.47 124.06) (end 104.14 125.73) (width 0.15) (layer F.Cu) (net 35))
 (segment (start 98.47 123.66) (end 103.34 123.66) (width 0.15) (layer F.Cu) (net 36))
 (segment (start 107.95 142.24) (end 105.41 144.78) (width 0.15) (layer B.Cu) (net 36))
 (segment (start 107.95 134.62) (end 107.95 142.24) (width 0.15) (layer B.Cu) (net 36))
 (segment (start 108.44 134.13) (end 107.95 134.62) (width 0.15) (layer B.Cu) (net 36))
 (segment (start 108.44 134.13) (end 111.43 134.13) (width 0.15) (layer B.Cu) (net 36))
 (via (at 105.41 144.78) (size 0.6) (drill 0.4) (layers F.Cu B.Cu) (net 36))
 (segment (start 105.41 125.73) (end 105.41 144.78) (width 0.15) (layer F.Cu) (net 36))
 (segment (start 103.34 123.66) (end 105.41 125.73) (width 0.15) (layer F.Cu) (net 36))
 (segment (start 98.47 123.26) (end 104.07 123.26) (width 0.15) (layer F.Cu) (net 37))
 (segment (start 109.71 136.67) (end 111.43 136.67) (width 0.15) (layer B.Cu) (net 37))
 (segment (start 106.68 144.78) (end 109.22 142.24) (width 0.15) (layer B.Cu) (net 37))
 (segment (start 109.22 137.16) (end 109.22 142.24) (width 0.15) (layer B.Cu) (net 37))
 (segment (start 109.71 136.67) (end 109.22 137.16) (width 0.15) (layer B.Cu) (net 37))
 (via (at 106.68 144.78) (size 0.6) (drill 0.4) (layers F.Cu B.Cu) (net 37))
 (segment (start 106.54 144.64) (end 106.68 144.78) (width 0.15) (layer F.Cu) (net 37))
 (segment (start 106.54 125.73) (end 106.54 144.64) (width 0.15) (layer F.Cu) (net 37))
 (segment (start 104.07 123.26) (end 106.54 125.73) (width 0.15) (layer F.Cu) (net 37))
 (segment (start 97.72 122.51) (end 97.72 120.72) (width 0.15) (layer F.Cu) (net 38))
 (segment (start 111.43 141.3) (end 111.43 139.21) (width 0.15) (layer B.Cu) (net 38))
 (segment (start 107.95 144.78) (end 111.43 141.3) (width 0.15) (layer B.Cu) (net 38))
 (via (at 107.95 144.78) (size 0.6) (drill 0.4) (layers F.Cu B.Cu) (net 38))
 (segment (start 107.95 125.73) (end 107.95 144.78) (width 0.15) (layer F.Cu) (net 38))
 (segment (start 102.87 120.65) (end 107.95 125.73) (width 0.15) (layer F.Cu) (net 38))
 (segment (start 97.79 120.65) (end 102.87 120.65) (width 0.15) (layer F.Cu) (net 38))
 (segment (start 97.72 120.72) (end 97.79 120.65) (width 0.15) (layer F.Cu) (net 38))
 (segment (start 59.71 136.66) (end 55.38 136.66) (width 0.15) (layer F.Cu) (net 41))
 (segment (start 55.38 136.66) (end 54.61 135.89) (width 0.15) (layer F.Cu) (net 41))
 (segment (start 95.25 119.21) (end 95.25 120.49506) (width 0.15) (layer F.Cu) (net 42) (status 400000))
 (segment (start 95.72 120.96506) (end 95.72 122.51) (width 0.15) (layer F.Cu) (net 42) (status 800000))
 (segment (start 95.25 120.49506) (end 95.72 120.96506) (width 0.15) (layer F.Cu) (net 42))
 (segment (start 55.92 134.66) (end 54.61 133.35) (width 0.15) (layer F.Cu) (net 42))
 (segment (start 59.71 134.66) (end 55.92 134.66) (width 0.15) (layer F.Cu) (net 42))
 (segment (start 95.73768 122.49232) (end 95.72 122.51) (width 0.15) (layer F.Cu) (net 42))
 (segment (start 101.6 124.46) (end 102.87 125.73) (width 0.15) (layer F.Cu) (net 6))
 (segment (start 102.87 125.73) (end 102.87 129.54) (width 0.15) (layer F.Cu) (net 6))
 (segment (start 102.87 129.54) (end 100.33 132.08) (width 0.15) (layer F.Cu) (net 6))
 (segment (start 100.33 132.08) (end 100.33 147.32) (width 0.15) (layer F.Cu) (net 6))
 (segment (start 97.79 132.08) (end 97.79 146.05) (width 0.15) (layer F.Cu) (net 43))
 (segment (start 100.33 129.54) (end 97.79 132.08) (width 0.15) (layer F.Cu) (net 43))
 (segment (start 97.79 146.05) (end 99.06 146.05) (width 0.15) (layer B.Cu) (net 43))
 (segment (start 102.87 142.24) (end 99.06 146.05) (width 0.15) (layer B.Cu) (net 43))
 (via (at 97.79 146.05) (size 0.6) (drill 0.4) (layers F.Cu B.Cu) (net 43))
 (segment (start 102.87 139.7) (end 102.87 142.24) (width 0.15) (layer B.Cu) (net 43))
 (segment (start 96.94672 119.22016) (end 96.94672 120.22328) (width 0.15) (layer F.Cu) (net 45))
 (segment (start 96.52 120.65) (end 96.52 122.51) (width 0.15) (layer F.Cu) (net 45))
 (segment (start 96.94672 120.22328) (end 96.52 120.65) (width 0.15) (layer F.Cu) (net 45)))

